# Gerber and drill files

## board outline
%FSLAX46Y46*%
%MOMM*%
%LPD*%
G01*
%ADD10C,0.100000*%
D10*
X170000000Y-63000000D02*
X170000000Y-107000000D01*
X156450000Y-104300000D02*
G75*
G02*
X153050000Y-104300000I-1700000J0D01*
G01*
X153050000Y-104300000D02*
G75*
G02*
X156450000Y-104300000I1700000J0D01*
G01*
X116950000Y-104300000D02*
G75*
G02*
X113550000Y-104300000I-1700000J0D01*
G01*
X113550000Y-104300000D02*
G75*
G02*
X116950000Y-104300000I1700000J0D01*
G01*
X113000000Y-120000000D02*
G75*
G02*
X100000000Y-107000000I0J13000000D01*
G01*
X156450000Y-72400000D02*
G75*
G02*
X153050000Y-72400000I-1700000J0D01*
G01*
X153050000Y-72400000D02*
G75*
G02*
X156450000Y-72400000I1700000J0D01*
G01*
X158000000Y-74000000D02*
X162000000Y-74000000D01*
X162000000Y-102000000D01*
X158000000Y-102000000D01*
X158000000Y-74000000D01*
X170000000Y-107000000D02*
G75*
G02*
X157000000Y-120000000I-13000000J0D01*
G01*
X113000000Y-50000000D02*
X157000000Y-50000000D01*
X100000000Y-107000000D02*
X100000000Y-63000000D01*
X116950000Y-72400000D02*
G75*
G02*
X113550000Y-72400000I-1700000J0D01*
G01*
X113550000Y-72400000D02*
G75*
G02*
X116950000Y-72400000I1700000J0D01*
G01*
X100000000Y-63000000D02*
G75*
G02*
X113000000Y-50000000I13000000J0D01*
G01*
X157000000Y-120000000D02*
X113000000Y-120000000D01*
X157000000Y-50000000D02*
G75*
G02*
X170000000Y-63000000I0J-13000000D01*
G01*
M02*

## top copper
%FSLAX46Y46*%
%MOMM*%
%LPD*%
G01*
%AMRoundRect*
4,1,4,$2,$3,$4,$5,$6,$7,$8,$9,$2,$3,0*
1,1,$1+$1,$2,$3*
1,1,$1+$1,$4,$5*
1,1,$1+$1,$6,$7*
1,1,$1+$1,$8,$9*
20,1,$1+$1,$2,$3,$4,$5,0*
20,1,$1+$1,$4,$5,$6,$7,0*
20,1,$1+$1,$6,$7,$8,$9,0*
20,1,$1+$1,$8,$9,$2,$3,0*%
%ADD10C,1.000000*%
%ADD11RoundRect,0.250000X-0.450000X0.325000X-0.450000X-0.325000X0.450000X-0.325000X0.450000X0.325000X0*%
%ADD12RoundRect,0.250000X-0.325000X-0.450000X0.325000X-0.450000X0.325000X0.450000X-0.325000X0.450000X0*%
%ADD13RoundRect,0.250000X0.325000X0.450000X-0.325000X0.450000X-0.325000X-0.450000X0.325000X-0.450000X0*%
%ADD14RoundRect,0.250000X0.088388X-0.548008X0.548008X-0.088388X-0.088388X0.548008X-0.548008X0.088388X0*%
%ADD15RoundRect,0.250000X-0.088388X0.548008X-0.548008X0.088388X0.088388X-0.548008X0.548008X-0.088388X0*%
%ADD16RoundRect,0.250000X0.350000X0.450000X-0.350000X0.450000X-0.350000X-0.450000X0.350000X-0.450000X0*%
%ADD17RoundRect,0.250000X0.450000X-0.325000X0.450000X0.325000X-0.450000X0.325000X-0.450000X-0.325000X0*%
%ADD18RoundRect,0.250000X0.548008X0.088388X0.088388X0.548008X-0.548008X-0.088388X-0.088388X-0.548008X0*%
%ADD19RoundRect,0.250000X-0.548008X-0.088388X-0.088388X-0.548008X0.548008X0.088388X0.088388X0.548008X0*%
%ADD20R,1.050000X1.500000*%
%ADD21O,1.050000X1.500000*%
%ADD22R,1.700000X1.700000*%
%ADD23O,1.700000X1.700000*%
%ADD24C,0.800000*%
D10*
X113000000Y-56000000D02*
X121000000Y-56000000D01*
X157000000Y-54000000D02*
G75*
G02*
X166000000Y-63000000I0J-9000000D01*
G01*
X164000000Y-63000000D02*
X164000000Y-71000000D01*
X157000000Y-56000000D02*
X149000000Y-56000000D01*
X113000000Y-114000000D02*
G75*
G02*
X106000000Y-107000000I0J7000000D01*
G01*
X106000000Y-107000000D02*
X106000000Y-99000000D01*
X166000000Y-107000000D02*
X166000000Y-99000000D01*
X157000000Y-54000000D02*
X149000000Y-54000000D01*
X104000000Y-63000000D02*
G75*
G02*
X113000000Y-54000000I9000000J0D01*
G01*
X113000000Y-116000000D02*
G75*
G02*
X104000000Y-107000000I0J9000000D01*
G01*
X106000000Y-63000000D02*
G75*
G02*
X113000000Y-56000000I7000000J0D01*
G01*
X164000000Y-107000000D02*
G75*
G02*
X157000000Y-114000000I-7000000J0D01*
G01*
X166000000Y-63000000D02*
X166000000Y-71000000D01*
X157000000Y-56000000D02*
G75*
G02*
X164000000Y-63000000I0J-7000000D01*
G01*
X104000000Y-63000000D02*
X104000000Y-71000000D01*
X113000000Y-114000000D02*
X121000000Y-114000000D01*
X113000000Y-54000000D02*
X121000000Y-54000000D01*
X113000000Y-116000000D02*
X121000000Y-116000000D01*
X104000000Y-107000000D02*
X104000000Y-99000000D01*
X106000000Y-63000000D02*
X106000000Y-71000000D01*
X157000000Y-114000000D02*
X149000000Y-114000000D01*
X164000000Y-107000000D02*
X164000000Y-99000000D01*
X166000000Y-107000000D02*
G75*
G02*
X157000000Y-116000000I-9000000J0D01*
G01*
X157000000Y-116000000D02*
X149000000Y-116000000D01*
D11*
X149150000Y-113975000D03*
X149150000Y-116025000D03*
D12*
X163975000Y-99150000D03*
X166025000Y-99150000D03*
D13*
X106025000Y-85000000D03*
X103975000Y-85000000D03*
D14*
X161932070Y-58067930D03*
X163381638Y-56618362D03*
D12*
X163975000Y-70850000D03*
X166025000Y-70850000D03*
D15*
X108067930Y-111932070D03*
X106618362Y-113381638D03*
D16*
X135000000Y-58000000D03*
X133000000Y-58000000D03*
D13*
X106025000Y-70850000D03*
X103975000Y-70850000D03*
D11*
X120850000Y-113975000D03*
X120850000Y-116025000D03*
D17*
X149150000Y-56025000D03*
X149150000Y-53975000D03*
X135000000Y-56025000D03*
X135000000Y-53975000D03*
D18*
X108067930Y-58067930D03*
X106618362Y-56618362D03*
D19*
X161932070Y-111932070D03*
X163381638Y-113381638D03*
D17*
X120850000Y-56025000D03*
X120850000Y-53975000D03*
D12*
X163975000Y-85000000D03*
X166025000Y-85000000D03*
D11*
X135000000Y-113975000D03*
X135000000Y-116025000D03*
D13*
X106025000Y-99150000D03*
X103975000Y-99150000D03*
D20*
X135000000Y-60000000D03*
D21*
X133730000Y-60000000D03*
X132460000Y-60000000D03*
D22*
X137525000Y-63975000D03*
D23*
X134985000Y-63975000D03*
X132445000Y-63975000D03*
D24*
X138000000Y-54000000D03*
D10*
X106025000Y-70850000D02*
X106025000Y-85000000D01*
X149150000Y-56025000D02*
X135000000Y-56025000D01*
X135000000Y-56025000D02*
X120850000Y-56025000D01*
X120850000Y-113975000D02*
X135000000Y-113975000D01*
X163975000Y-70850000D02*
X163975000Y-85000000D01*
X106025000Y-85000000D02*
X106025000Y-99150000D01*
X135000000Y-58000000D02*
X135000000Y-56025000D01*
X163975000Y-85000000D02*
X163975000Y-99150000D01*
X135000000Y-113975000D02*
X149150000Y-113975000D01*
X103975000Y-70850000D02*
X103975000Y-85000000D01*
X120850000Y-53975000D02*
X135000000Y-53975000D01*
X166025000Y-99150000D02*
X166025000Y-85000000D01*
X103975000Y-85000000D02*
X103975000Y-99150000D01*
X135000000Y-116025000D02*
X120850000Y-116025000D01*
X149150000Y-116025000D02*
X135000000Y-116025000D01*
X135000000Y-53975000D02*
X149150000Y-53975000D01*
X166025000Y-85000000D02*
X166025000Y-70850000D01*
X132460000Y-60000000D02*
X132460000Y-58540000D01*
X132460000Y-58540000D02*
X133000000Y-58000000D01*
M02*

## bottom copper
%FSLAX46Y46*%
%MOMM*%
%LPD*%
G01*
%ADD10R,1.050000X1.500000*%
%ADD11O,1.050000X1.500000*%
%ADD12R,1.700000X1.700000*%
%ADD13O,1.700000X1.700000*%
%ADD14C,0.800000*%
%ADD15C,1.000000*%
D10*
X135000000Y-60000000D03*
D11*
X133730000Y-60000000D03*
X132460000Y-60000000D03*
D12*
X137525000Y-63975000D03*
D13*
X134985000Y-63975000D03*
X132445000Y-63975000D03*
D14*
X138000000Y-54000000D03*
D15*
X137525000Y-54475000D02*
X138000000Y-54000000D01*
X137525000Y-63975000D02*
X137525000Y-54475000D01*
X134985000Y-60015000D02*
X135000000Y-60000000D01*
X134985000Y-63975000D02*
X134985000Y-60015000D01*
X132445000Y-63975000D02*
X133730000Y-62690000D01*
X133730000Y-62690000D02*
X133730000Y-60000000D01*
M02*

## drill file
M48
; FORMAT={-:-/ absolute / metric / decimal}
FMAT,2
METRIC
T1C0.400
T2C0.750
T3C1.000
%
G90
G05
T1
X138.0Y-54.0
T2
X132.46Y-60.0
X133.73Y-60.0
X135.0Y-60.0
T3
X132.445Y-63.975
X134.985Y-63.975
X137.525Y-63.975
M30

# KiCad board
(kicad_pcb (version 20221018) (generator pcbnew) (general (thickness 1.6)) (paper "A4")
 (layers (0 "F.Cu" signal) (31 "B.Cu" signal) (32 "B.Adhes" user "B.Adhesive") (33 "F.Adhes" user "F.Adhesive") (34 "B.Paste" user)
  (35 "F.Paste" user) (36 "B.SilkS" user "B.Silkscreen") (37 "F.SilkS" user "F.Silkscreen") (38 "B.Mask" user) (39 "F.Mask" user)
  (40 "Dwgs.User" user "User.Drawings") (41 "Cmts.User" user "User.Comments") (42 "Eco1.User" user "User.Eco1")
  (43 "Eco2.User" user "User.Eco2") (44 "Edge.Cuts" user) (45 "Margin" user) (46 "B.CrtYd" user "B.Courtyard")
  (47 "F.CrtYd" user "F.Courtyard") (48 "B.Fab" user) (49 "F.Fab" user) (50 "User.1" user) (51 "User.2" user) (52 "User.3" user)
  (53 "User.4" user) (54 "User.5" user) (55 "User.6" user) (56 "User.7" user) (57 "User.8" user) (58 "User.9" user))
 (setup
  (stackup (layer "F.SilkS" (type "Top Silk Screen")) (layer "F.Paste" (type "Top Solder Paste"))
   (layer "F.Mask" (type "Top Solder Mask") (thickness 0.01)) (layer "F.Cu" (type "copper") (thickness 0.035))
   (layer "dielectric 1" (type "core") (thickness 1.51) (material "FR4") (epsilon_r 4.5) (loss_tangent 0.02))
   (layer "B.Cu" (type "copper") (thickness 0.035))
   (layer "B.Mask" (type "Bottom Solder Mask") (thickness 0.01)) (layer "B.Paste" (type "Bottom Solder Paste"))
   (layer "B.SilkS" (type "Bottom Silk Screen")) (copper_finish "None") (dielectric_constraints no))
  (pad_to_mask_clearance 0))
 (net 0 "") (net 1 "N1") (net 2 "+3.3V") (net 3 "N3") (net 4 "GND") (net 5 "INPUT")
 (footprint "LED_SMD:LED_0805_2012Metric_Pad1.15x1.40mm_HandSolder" (layer "F.Cu") (at 149.15 115 -90)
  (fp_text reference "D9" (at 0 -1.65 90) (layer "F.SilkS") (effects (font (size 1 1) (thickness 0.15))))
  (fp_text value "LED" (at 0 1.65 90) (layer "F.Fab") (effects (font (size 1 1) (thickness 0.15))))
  (pad "1" smd roundrect (at -1.025 0 270) (size 1.15 1.4) (layers "F.Cu" "F.Paste" "F.Mask") (roundrect_rratio 0.2173913043) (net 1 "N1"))
  (pad "2" smd roundrect (at 1.025 0 270) (size 1.15 1.4) (layers "F.Cu" "F.Paste" "F.Mask") (roundrect_rratio 0.2173913043) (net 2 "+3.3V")))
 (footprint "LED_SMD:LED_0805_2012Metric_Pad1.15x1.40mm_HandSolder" (layer "F.Cu") (at 165 99.15)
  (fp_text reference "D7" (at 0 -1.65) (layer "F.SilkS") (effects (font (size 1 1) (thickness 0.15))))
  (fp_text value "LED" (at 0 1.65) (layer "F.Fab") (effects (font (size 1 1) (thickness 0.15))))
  (pad "1" smd roundrect (at -1.025 0) (size 1.15 1.4) (layers "F.Cu" "F.Paste" "F.Mask") (roundrect_rratio 0.2173913043) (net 1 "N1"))
  (pad "2" smd roundrect (at 1.025 0) (size 1.15 1.4) (layers "F.Cu" "F.Paste" "F.Mask") (roundrect_rratio 0.2173913043) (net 2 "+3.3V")))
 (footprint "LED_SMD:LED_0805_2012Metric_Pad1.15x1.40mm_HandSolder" (layer "F.Cu") (at 105 85 180)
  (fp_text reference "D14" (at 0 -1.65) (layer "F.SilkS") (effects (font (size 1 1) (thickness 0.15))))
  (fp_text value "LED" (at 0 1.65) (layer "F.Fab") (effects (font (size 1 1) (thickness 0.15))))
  (pad "1" smd roundrect (at -1.025 0 180) (size 1.15 1.4) (layers "F.Cu" "F.Paste" "F.Mask") (roundrect_rratio 0.2173913043) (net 1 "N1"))
  (pad "2" smd roundrect (at 1.025 0 180) (size 1.15 1.4) (layers "F.Cu" "F.Paste" "F.Mask") (roundrect_rratio 0.2173913043) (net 2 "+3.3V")))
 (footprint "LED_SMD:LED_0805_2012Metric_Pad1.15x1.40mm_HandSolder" (layer "F.Cu") (at 162.656854 57.343146 45)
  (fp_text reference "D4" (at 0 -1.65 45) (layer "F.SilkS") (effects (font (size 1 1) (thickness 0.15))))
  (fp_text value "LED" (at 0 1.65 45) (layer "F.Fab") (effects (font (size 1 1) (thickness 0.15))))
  (pad "1" smd roundrect (at -1.025 0 45) (size 1.15 1.4) (layers "F.Cu" "F.Paste" "F.Mask") (roundrect_rratio 0.2173913043) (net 1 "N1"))
  (pad "2" smd roundrect (at 1.025 0 45) (size 1.15 1.4) (layers "F.Cu" "F.Paste" "F.Mask") (roundrect_rratio 0.2173913043) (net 2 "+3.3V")))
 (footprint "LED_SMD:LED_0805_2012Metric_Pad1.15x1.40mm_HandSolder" (layer "F.Cu") (at 165 70.85)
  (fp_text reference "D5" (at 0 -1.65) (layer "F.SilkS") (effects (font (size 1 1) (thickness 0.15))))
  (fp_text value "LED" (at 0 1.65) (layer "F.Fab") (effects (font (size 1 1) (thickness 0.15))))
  (pad "1" smd roundrect (at -1.025 0) (size 1.15 1.4) (layers "F.Cu" "F.Paste" "F.Mask") (roundrect_rratio 0.2173913043) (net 1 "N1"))
  (pad "2" smd roundrect (at 1.025 0) (size 1.15 1.4) (layers "F.Cu" "F.Paste" "F.Mask") (roundrect_rratio 0.2173913043) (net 2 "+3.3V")))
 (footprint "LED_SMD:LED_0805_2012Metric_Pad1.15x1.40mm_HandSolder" (layer "F.Cu") (at 107.343146 112.656854 -135)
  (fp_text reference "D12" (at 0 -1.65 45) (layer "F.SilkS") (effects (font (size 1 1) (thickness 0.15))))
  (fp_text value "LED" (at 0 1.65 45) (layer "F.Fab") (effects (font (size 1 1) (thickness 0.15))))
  (pad "1" smd roundrect (at -1.025 0 225) (size 1.15 1.4) (layers "F.Cu" "F.Paste" "F.Mask") (roundrect_rratio 0.2173913043) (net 1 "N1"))
  (pad "2" smd roundrect (at 1.025 0 225) (size 1.15 1.4) (layers "F.Cu" "F.Paste" "F.Mask") (roundrect_rratio 0.2173913043) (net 2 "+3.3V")))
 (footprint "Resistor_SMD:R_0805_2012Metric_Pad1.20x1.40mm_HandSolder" (layer "F.Cu") (at 134 58 180)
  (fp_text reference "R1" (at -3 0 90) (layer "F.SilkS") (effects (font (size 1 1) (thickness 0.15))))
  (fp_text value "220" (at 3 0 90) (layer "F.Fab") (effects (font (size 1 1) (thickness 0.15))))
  (pad "1" smd roundrect (at -1 0 180) (size 1.2 1.4) (layers "F.Cu" "F.Paste" "F.Mask") (roundrect_rratio 0.2083333333) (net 1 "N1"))
  (pad "2" smd roundrect (at 1 0 180) (size 1.2 1.4) (layers "F.Cu" "F.Paste" "F.Mask") (roundrect_rratio 0.2083333333) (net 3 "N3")))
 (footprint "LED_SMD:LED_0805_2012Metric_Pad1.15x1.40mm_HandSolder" (layer "F.Cu") (at 105 70.85 180)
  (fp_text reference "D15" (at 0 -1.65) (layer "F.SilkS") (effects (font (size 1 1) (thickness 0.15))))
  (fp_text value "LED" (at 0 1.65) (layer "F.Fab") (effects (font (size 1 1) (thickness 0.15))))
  (pad "1" smd roundrect (at -1.025 0 180) (size 1.15 1.4) (layers "F.Cu" "F.Paste" "F.Mask") (roundrect_rratio 0.2173913043) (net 1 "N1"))
  (pad "2" smd roundrect (at 1.025 0 180) (size 1.15 1.4) (layers "F.Cu" "F.Paste" "F.Mask") (roundrect_rratio 0.2173913043) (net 2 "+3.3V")))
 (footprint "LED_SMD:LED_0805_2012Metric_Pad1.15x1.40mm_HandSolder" (layer "F.Cu") (at 120.85 115 -90)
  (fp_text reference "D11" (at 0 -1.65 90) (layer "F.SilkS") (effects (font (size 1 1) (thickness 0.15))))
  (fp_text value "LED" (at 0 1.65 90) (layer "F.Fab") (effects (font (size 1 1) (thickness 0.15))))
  (pad "1" smd roundrect (at -1.025 0 270) (size 1.15 1.4) (layers "F.Cu" "F.Paste" "F.Mask") (roundrect_rratio 0.2173913043) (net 1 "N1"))
  (pad "2" smd roundrect (at 1.025 0 270) (size 1.15 1.4) (layers "F.Cu" "F.Paste" "F.Mask") (roundrect_rratio 0.2173913043) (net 2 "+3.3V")))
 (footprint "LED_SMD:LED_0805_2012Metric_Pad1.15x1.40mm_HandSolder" (layer "F.Cu") (at 149.15 55 90)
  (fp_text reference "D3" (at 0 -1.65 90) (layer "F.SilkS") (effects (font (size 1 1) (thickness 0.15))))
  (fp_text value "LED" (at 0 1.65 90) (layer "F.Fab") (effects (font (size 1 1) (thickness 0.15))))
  (pad "1" smd roundrect (at -1.025 0 90) (size 1.15 1.4) (layers "F.Cu" "F.Paste" "F.Mask") (roundrect_rratio 0.2173913043) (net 1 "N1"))
  (pad "2" smd roundrect (at 1.025 0 90) (size 1.15 1.4) (layers "F.Cu" "F.Paste" "F.Mask") (roundrect_rratio 0.2173913043) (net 2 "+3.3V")))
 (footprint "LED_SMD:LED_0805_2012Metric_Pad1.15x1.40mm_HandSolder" (layer "F.Cu") (at 135 55 90)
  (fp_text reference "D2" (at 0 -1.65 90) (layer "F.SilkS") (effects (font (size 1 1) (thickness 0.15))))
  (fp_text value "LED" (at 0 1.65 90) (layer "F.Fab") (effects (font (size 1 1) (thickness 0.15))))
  (pad "1" smd roundrect (at -1.025 0 90) (size 1.15 1.4) (layers "F.Cu" "F.Paste" "F.Mask") (roundrect_rratio 0.2173913043) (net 1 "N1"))
  (pad "2" smd roundrect (at 1.025 0 90) (size 1.15 1.4) (layers "F.Cu" "F.Paste" "F.Mask") (roundrect_rratio 0.2173913043) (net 2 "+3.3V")))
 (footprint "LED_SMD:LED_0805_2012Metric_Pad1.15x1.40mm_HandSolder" (layer "F.Cu") (at 107.343146 57.343146 135)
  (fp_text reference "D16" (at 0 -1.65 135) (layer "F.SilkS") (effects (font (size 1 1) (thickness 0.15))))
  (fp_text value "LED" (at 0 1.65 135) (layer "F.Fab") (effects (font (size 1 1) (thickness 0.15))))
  (pad "1" smd roundrect (at -1.025 0 135) (size 1.15 1.4) (layers "F.Cu" "F.Paste" "F.Mask") (roundrect_rratio 0.2173913043) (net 1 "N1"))
  (pad "2" smd roundrect (at 1.025 0 135) (size 1.15 1.4) (layers "F.Cu" "F.Paste" "F.Mask") (roundrect_rratio 0.2173913043) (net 2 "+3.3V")))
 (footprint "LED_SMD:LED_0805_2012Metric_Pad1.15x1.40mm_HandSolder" (layer "F.Cu") (at 162.656854 112.656854 -45)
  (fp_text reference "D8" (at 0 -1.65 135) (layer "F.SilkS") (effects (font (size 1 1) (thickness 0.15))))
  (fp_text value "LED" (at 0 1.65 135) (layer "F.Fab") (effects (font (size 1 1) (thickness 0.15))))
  (pad "1" smd roundrect (at -1.025 0 315) (size 1.15 1.4) (layers "F.Cu" "F.Paste" "F.Mask") (roundrect_rratio 0.2173913043) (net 1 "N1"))
  (pad "2" smd roundrect (at 1.025 0 315) (size 1.15 1.4) (layers "F.Cu" "F.Paste" "F.Mask") (roundrect_rratio 0.2173913043) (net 2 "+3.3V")))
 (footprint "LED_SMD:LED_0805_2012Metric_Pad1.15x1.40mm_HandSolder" (layer "F.Cu") (at 120.85 55 90)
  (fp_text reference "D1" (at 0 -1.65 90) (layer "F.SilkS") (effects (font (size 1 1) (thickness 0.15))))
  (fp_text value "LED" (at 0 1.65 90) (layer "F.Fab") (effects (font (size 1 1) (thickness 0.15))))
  (pad "1" smd roundrect (at -1.025 0 90) (size 1.15 1.4) (layers "F.Cu" "F.Paste" "F.Mask") (roundrect_rratio 0.2173913043) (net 1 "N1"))
  (pad "2" smd roundrect (at 1.025 0 90) (size 1.15 1.4) (layers "F.Cu" "F.Paste" "F.Mask") (roundrect_rratio 0.2173913043) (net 2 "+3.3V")))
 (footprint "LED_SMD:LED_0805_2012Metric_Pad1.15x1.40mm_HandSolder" (layer "F.Cu") (at 165 85)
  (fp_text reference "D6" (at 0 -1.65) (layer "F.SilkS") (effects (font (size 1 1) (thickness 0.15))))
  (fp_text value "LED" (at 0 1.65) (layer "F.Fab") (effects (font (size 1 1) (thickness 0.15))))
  (pad "1" smd roundrect (at -1.025 0) (size 1.15 1.4) (layers "F.Cu" "F.Paste" "F.Mask") (roundrect_rratio 0.2173913043) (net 1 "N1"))
  (pad "2" smd roundrect (at 1.025 0) (size 1.15 1.4) (layers "F.Cu" "F.Paste" "F.Mask") (roundrect_rratio 0.2173913043) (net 2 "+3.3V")))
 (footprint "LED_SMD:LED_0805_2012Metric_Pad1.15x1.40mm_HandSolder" (layer "F.Cu") (at 135 115 -90)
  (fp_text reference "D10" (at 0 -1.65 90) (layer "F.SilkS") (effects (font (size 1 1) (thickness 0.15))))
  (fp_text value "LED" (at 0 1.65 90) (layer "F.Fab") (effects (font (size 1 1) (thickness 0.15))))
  (pad "1" smd roundrect (at -1.025 0 270) (size 1.15 1.4) (layers "F.Cu" "F.Paste" "F.Mask") (roundrect_rratio 0.2173913043) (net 1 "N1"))
  (pad "2" smd roundrect (at 1.025 0 270) (size 1.15 1.4) (layers "F.Cu" "F.Paste" "F.Mask") (roundrect_rratio 0.2173913043) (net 2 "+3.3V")))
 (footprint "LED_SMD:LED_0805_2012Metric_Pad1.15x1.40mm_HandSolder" (layer "F.Cu") (at 105 99.15 180)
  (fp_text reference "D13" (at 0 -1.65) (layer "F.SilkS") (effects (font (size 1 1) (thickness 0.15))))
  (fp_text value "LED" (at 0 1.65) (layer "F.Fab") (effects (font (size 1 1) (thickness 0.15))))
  (pad "1" smd roundrect (at -1.025 0 180) (size 1.15 1.4) (layers "F.Cu" "F.Paste" "F.Mask") (roundrect_rratio 0.2173913043) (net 1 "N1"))
  (pad "2" smd roundrect (at 1.025 0 180) (size 1.15 1.4) (layers "F.Cu" "F.Paste" "F.Mask") (roundrect_rratio 0.2173913043) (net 2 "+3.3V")))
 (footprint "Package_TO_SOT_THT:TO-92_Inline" (layer "B.Cu") (at 135 60 180)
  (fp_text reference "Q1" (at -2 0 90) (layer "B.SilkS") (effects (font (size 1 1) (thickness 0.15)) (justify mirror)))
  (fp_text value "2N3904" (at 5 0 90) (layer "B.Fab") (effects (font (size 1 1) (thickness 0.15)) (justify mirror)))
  (pad "1" thru_hole rect (at 0 0 180) (size 1.05 1.5) (drill 0.75) (layers "*.Cu" "*.Mask") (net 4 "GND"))
  (pad "2" thru_hole oval (at 1.27 0 180) (size 1.05 1.5) (drill 0.75) (layers "*.Cu" "*.Mask") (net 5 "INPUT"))
  (pad "3" thru_hole oval (at 2.54 0 180) (size 1.05 1.5) (drill 0.75) (layers "*.Cu" "*.Mask") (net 3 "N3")))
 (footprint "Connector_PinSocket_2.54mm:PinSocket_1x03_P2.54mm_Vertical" (layer "B.Cu") (at 137.525 63.975 90)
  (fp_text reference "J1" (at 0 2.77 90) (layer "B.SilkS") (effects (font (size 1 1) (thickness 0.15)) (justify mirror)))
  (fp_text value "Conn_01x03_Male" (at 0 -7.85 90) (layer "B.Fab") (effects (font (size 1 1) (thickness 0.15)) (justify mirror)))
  (pad "1" thru_hole rect (at 0 0 90) (size 1.7 1.7) (drill 1) (layers "*.Cu" "*.Mask") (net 2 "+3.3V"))
  (pad "2" thru_hole oval (at 0 -2.54 90) (size 1.7 1.7) (drill 1) (layers "*.Cu" "*.Mask") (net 4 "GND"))
  (pad "3" thru_hole oval (at 0 -5.08 90) (size 1.7 1.7) (drill 1) (layers "*.Cu" "*.Mask") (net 5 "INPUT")))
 (gr_line (start 113 56) (end 121 56) (stroke (width 1) (type solid)) (layer "F.Cu"))
 (gr_arc (start 157 54) (mid 163.363961 56.636039) (end 166 63) (stroke (width 1) (type solid)) (layer "F.Cu"))
 (gr_line (start 164 63) (end 164 71) (stroke (width 1) (type solid)) (layer "F.Cu"))
 (gr_line (start 157 56) (end 149 56) (stroke (width 1) (type solid)) (layer "F.Cu"))
 (gr_arc (start 113 114) (mid 108.050253 111.949747) (end 106 107) (stroke (width 1) (type solid)) (layer "F.Cu"))
 (gr_line (start 106 107) (end 106 99) (stroke (width 1) (type solid)) (layer "F.Cu"))
 (gr_line (start 166 107) (end 166 99) (stroke (width 1) (type solid)) (layer "F.Cu"))
 (gr_line (start 157 54) (end 149 54) (stroke (width 1) (type solid)) (layer "F.Cu"))
 (gr_arc (start 104 63) (mid 106.636039 56.636039) (end 113 54) (stroke (width 1) (type solid)) (layer "F.Cu"))
 (gr_arc (start 113 116) (mid 106.636039 113.363961) (end 104 107) (stroke (width 1) (type solid)) (layer "F.Cu"))
 (gr_arc (start 106 63) (mid 108.050253 58.050253) (end 113 56) (stroke (width 1) (type solid)) (layer "F.Cu"))
 (gr_arc (start 164 107) (mid 161.949747 111.949747) (end 157 114) (stroke (width 1) (type solid)) (layer "F.Cu"))
 (gr_line (start 166 63) (end 166 71) (stroke (width 1) (type solid)) (layer "F.Cu"))
 (gr_arc (start 157 56) (mid 161.949747 58.050253) (end 164 63) (stroke (width 1) (type solid)) (layer "F.Cu"))
 (gr_line (start 104 63) (end 104 71) (stroke (width 1) (type solid)) (layer "F.Cu"))
 (gr_line (start 113 114) (end 121 114) (stroke (width 1) (type solid)) (layer "F.Cu"))
 (gr_line (start 113 54) (end 121 54) (stroke (width 1) (type solid)) (layer "F.Cu"))
 (gr_line (start 113 116) (end 121 116) (stroke (width 1) (type solid)) (layer "F.Cu"))
 (gr_line (start 104 107) (end 104 99) (stroke (width 1) (type solid)) (layer "F.Cu"))
 (gr_line (start 106 63) (end 106 71) (stroke (width 1) (type solid)) (layer "F.Cu"))
 (gr_line (start 157 114) (end 149 114) (stroke (width 1) (type solid)) (layer "F.Cu"))
 (gr_line (start 164 107) (end 164 99) (stroke (width 1) (type solid)) (layer "F.Cu"))
 (gr_arc (start 166 107) (mid 163.363961 113.363961) (end 157 116) (stroke (width 1) (type solid)) (layer "F.Cu"))
 (gr_line (start 157 116) (end 149 116) (stroke (width 1) (type solid)) (layer "F.Cu"))
 (gr_line (start 170 63) (end 170 107) (stroke (width 0.1) (type solid)) (layer "Edge.Cuts"))
 (gr_circle (center 154.75 104.3) (end 156.45 104.3) (stroke (width 0.1) (type solid)) (fill none) (layer "Edge.Cuts"))
 (gr_circle (center 115.25 104.3) (end 116.95 104.3) (stroke (width 0.1) (type solid)) (fill none) (layer "Edge.Cuts"))
 (gr_arc (start 113 120) (mid 103.807612 116.192388) (end 100 107) (stroke (width 0.1) (type solid)) (layer "Edge.Cuts"))
 (gr_circle (center 154.75 72.4) (end 156.45 72.4) (stroke (width 0.1) (type solid)) (fill none) (layer "Edge.Cuts"))
 (gr_rect (start 158 74) (end 162 102) (stroke (width 0.1) (type solid)) (fill none) (layer "Edge.Cuts"))
 (gr_arc (start 170 107) (mid 166.192388 116.192388) (end 157 120) (stroke (width 0.1) (type solid)) (layer "Edge.Cuts"))
 (gr_line (start 113 50) (end 157 50) (stroke (width 0.1) (type solid)) (layer "Edge.Cuts"))
 (gr_line (start 100 107) (end 100 63) (stroke (width 0.1) (type solid)) (layer "Edge.Cuts"))
 (gr_circle (center 115.25 72.4) (end 116.95 72.4) (stroke (width 0.1) (type solid)) (fill none) (layer "Edge.Cuts"))
 (gr_arc (start 100 63) (mid 103.807612 53.807612) (end 113 50) (stroke (width 0.1) (type solid)) (layer "Edge.Cuts"))
 (gr_line (start 157 120) (end 113 120) (stroke (width 0.1) (type solid)) (layer "Edge.Cuts"))
 (gr_arc (start 157 50) (mid 166.192388 53.807612) (end 170 63) (stroke (width 0.1) (type solid)) (layer "Edge.Cuts"))
 (segment (start 106.025 70.85) (end 106.025 85) (width 1) (layer "F.Cu") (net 1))
 (segment (start 149.15 56.025) (end 135 56.025) (width 1) (layer "F.Cu") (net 1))
 (segment (start 135 56.025) (end 120.85 56.025) (width 1) (layer "F.Cu") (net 1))
 (segment (start 120.85 113.975) (end 135 113.975) (width 1) (layer "F.Cu") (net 1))
 (segment (start 163.975 70.85) (end 163.975 85) (width 1) (layer "F.Cu") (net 1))
 (segment (start 106.025 85) (end 106.025 99.15) (width 1) (layer "F.Cu") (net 1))
 (segment (start 135 58) (end 135 56.025) (width 1) (layer "F.Cu") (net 1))
 (segment (start 163.975 85) (end 163.975 99.15) (width 1) (layer "F.Cu") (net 1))
 (segment (start 135 113.975) (end 149.15 113.975) (width 1) (layer "F.Cu") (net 1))
 (segment (start 103.975 70.85) (end 103.975 85) (width 1) (layer "F.Cu") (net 2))
 (segment (start 120.85 53.975) (end 135 53.975) (width 1) (layer "F.Cu") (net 2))
 (segment (start 166.025 99.15) (end 166.025 85) (width 1) (layer "F.Cu") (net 2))
 (segment (start 103.975 85) (end 103.975 99.15) (width 1) (layer "F.Cu") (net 2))
 (segment (start 135 116.025) (end 120.85 116.025) (width 1) (layer "F.Cu") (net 2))
 (segment (start 149.15 116.025) (end 135 116.025) (width 1) (layer "F.Cu") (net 2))
 (segment (start 135 53.975) (end 149.15 53.975) (width 1) (layer "F.Cu") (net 2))
 (segment (start 166.025 85) (end 166.025 70.85) (width 1) (layer "F.Cu") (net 2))
 (via (at 138 54) (size 0.8) (drill 0.4) (layers "F.Cu" "B.Cu") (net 2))
 (segment (start 137.525 54.475) (end 138 54) (width 1) (layer "B.Cu") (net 2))
 (segment (start 137.525 63.975) (end 137.525 54.475) (width 1) (layer "B.Cu") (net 2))
 (segment (start 134.985 60.015) (end 135 60) (width 1) (layer "B.Cu") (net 4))
 (segment (start 134.985 63.975) (end 134.985 60.015) (width 1) (layer "B.Cu") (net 4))
 (segment (start 132.445 63.975) (end 133.73 62.69) (width 1) (layer "B.Cu") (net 5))
 (segment (start 133.73 62.69) (end 133.73 60) (width 1) (layer "B.Cu") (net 5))
 (segment (start 132.46 60) (end 132.46 58.54) (width 1) (layer "F.Cu") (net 3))
 (segment (start 132.46 58.54) (end 133 58) (width 1) (layer "F.Cu") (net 3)))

